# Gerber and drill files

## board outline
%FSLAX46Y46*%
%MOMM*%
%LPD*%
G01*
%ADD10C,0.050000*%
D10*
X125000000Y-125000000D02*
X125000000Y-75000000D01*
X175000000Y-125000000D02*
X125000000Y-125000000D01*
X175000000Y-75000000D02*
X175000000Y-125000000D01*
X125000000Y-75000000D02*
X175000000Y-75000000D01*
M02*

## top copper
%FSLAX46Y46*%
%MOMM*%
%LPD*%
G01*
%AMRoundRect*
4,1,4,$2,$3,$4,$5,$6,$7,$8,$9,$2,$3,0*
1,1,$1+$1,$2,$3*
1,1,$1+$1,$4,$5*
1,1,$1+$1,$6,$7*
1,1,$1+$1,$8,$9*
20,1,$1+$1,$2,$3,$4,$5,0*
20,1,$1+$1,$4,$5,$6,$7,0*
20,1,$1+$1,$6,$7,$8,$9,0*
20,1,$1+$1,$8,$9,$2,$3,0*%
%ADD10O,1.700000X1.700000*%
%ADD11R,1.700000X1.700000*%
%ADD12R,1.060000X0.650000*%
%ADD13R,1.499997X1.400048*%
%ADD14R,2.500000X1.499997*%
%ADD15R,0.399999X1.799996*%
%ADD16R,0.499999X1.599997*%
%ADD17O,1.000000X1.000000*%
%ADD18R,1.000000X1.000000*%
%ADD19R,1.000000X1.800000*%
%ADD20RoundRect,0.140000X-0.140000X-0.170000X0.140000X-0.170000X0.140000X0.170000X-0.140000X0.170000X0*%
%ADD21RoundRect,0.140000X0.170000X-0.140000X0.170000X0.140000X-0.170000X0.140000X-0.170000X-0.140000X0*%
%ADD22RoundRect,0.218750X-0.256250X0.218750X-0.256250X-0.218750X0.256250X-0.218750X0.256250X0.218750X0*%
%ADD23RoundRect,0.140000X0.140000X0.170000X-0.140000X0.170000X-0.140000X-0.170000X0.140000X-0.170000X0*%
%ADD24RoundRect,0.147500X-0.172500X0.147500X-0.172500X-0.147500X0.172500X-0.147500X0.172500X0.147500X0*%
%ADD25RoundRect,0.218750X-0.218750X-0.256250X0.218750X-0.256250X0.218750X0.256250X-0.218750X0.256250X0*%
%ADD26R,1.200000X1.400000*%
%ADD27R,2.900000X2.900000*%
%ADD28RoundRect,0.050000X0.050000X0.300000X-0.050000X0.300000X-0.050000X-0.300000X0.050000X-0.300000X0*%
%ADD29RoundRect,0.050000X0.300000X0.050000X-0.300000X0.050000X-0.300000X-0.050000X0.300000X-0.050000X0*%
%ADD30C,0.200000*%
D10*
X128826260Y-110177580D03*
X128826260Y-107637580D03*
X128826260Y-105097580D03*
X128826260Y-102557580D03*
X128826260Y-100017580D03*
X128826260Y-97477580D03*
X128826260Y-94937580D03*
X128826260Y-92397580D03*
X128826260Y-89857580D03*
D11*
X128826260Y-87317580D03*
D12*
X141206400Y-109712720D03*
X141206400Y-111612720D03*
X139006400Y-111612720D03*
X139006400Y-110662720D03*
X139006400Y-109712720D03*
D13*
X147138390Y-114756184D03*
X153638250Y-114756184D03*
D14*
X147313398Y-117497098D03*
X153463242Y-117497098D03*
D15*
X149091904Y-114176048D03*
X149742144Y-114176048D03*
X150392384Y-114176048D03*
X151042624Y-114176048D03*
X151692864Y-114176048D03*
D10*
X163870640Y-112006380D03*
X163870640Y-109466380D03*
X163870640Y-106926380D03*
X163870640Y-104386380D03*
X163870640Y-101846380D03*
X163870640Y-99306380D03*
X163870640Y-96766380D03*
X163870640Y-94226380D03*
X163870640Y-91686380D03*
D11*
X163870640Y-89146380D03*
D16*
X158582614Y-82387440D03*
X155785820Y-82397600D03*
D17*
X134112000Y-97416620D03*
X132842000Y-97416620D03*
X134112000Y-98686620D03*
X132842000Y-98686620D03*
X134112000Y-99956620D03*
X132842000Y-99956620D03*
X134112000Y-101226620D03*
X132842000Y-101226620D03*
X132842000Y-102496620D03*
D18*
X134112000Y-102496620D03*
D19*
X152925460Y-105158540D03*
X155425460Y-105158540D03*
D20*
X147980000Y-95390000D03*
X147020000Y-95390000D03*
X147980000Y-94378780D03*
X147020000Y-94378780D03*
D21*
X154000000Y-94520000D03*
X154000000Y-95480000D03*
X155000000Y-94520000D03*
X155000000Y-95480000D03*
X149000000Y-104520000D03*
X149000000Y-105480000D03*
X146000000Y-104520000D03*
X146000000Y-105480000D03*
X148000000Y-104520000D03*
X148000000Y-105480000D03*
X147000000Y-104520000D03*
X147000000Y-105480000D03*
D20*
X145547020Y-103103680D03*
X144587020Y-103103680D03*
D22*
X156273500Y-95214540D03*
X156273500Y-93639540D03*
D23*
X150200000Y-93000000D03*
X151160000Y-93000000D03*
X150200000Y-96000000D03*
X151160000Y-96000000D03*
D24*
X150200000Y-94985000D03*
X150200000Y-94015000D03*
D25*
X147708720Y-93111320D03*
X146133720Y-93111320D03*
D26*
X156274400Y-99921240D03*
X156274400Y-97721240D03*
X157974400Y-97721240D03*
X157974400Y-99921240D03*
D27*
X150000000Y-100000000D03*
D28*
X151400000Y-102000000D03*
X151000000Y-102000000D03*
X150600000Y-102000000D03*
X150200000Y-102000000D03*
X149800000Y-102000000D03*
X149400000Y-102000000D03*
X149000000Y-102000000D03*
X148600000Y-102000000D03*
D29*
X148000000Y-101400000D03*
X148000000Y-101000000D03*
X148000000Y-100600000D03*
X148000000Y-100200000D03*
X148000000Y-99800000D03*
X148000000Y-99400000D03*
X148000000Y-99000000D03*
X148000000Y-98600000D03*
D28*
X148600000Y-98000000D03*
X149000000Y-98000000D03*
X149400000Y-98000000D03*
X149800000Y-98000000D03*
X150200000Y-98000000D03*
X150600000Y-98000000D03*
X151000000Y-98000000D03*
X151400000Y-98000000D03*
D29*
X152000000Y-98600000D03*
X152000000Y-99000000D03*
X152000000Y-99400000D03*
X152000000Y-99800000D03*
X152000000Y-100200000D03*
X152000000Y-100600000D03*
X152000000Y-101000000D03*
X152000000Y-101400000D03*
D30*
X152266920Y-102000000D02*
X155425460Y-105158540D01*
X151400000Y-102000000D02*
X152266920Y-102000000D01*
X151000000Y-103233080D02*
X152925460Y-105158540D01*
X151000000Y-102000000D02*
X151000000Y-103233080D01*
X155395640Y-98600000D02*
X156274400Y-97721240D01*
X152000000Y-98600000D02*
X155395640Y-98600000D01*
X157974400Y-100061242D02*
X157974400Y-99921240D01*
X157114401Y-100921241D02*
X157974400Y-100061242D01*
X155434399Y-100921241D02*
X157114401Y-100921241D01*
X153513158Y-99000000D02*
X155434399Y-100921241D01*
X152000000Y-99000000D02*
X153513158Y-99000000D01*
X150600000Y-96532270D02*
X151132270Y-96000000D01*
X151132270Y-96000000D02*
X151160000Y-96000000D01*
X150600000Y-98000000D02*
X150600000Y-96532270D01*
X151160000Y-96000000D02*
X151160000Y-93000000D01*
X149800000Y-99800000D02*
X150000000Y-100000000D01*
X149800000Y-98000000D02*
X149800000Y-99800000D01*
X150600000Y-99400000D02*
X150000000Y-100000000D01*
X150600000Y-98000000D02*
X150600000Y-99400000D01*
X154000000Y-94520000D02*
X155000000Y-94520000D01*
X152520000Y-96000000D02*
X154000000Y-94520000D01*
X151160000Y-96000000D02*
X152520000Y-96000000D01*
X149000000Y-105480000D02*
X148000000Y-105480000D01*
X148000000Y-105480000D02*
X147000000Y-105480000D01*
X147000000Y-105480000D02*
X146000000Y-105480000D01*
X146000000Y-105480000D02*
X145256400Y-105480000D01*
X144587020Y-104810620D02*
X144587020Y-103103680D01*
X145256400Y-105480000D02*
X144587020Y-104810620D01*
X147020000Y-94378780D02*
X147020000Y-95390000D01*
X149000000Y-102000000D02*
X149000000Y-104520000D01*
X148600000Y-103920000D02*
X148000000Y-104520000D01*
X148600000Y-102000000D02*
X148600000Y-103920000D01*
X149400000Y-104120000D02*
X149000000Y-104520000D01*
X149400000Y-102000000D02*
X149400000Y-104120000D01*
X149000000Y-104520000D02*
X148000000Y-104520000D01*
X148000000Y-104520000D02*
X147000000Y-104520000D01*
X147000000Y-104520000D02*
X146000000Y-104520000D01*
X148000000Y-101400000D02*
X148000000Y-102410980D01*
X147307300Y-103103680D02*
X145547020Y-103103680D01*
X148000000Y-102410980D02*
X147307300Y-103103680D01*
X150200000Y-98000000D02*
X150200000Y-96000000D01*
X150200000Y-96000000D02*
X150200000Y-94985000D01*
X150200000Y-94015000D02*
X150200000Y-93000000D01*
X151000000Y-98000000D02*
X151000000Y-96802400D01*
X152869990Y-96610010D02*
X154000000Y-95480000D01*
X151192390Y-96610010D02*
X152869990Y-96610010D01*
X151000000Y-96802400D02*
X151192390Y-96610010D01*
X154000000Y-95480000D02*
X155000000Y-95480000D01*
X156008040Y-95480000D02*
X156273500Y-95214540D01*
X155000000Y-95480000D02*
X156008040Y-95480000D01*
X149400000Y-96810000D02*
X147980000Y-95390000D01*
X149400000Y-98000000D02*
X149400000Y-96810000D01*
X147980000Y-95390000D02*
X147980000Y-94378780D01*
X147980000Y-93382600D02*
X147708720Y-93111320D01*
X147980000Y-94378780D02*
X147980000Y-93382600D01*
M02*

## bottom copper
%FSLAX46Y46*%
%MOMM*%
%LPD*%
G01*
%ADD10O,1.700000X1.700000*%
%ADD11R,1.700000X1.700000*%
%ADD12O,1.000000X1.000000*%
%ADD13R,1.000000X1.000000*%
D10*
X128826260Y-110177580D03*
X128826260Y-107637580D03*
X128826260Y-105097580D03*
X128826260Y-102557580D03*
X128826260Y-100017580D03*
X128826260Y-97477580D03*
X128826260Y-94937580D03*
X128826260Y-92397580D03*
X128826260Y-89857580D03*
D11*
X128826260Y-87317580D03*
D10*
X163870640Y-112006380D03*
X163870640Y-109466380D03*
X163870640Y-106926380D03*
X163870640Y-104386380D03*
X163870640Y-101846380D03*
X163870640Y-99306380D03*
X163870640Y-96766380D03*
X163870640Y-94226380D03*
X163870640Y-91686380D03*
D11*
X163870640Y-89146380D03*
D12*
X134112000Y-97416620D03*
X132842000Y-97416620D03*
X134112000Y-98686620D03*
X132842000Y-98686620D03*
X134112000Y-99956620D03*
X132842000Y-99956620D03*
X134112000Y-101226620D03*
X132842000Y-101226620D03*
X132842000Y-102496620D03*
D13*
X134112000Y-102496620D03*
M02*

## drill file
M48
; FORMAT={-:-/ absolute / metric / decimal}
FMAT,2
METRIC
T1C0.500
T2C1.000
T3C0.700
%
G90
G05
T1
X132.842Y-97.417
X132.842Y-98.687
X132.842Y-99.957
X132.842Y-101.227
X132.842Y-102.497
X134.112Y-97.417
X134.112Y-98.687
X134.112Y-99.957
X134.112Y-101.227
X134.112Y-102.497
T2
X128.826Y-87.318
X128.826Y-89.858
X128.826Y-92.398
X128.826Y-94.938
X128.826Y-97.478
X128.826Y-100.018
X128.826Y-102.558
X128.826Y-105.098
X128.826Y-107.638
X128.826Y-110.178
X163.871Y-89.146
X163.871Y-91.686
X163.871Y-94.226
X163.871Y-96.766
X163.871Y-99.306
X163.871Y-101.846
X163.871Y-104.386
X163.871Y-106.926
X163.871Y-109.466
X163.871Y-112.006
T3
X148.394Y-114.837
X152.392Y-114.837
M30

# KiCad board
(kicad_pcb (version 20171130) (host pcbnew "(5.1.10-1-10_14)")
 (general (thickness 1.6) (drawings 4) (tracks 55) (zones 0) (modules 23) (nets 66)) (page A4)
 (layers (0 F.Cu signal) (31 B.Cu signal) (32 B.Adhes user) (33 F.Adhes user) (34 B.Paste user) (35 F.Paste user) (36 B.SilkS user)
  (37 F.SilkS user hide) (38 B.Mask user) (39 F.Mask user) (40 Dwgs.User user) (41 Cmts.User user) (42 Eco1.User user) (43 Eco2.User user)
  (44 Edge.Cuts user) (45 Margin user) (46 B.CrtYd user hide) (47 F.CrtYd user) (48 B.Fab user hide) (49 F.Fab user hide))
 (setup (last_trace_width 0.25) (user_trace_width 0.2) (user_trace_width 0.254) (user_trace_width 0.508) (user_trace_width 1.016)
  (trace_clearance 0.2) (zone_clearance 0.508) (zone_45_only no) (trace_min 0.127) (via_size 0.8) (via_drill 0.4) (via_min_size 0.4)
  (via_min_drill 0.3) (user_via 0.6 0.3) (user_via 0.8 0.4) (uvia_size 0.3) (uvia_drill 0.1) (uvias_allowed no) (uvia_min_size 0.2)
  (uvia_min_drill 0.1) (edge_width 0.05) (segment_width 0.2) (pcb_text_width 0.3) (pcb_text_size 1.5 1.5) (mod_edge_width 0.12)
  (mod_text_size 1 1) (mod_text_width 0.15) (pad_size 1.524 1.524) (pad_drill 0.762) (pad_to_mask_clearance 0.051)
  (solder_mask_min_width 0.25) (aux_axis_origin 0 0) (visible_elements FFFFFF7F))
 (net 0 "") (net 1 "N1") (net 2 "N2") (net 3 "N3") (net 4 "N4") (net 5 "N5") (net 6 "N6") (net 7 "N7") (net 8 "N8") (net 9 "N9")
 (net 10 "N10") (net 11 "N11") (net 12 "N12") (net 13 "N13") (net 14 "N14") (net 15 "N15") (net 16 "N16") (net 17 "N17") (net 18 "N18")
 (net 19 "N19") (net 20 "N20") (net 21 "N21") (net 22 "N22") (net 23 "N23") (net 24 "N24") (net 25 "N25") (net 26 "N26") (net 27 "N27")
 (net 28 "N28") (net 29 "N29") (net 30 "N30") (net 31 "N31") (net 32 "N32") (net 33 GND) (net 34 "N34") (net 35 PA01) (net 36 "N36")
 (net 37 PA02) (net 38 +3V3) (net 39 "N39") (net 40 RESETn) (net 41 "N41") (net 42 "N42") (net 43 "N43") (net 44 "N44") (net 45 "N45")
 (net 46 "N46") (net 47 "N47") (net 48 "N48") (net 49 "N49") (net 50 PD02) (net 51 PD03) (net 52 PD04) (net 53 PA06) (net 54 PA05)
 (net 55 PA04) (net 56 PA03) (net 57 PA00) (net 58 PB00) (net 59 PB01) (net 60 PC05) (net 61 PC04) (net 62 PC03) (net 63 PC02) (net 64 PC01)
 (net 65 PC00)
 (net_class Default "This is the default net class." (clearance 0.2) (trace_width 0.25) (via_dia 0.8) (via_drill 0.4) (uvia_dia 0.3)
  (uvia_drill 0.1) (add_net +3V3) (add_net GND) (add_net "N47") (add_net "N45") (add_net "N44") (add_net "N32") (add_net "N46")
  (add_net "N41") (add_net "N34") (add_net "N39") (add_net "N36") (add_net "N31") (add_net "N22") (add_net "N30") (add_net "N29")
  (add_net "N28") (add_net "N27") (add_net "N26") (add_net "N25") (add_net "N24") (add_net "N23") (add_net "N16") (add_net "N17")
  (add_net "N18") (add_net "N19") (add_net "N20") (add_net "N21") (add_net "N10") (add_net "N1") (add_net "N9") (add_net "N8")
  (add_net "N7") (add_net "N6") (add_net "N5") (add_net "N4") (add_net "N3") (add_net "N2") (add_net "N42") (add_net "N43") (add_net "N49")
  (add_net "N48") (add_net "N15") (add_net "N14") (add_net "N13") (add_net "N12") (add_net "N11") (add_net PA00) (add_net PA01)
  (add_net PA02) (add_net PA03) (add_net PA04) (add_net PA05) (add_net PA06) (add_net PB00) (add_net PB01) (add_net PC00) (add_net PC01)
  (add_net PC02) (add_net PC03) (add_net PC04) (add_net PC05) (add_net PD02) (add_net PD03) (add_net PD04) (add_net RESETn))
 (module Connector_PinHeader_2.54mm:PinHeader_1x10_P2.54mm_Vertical (layer F.Cu) (at 128.82626 87.31758)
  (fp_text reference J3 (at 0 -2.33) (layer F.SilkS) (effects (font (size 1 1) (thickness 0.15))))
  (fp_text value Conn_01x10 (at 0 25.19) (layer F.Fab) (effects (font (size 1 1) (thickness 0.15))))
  (pad 10 thru_hole oval (at 0 22.86) (size 1.7 1.7) (drill 1) (layers *.Cu *.Mask) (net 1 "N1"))
  (pad 9 thru_hole oval (at 0 20.32) (size 1.7 1.7) (drill 1) (layers *.Cu *.Mask) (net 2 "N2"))
  (pad 8 thru_hole oval (at 0 17.78) (size 1.7 1.7) (drill 1) (layers *.Cu *.Mask) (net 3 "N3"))
  (pad 7 thru_hole oval (at 0 15.24) (size 1.7 1.7) (drill 1) (layers *.Cu *.Mask) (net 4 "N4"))
  (pad 6 thru_hole oval (at 0 12.7) (size 1.7 1.7) (drill 1) (layers *.Cu *.Mask) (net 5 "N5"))
  (pad 5 thru_hole oval (at 0 10.16) (size 1.7 1.7) (drill 1) (layers *.Cu *.Mask) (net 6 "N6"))
  (pad 4 thru_hole oval (at 0 7.62) (size 1.7 1.7) (drill 1) (layers *.Cu *.Mask) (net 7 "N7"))
  (pad 3 thru_hole oval (at 0 5.08) (size 1.7 1.7) (drill 1) (layers *.Cu *.Mask) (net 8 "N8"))
  (pad 2 thru_hole oval (at 0 2.54) (size 1.7 1.7) (drill 1) (layers *.Cu *.Mask) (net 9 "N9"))
  (pad 1 thru_hole rect (at 0 0) (size 1.7 1.7) (drill 1) (layers *.Cu *.Mask) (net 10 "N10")))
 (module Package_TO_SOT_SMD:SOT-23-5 (layer F.Cu) (at 140.1064 110.66272)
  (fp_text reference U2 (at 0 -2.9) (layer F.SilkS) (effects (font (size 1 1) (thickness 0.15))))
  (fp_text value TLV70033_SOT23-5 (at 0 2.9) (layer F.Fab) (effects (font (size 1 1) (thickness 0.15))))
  (pad 5 smd rect (at 1.1 -0.95) (size 1.06 0.65) (layers F.Cu F.Paste F.Mask) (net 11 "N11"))
  (pad 4 smd rect (at 1.1 0.95) (size 1.06 0.65) (layers F.Cu F.Paste F.Mask) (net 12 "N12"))
  (pad 3 smd rect (at -1.1 0.95) (size 1.06 0.65) (layers F.Cu F.Paste F.Mask) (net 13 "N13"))
  (pad 2 smd rect (at -1.1 0) (size 1.06 0.65) (layers F.Cu F.Paste F.Mask) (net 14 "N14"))
  (pad 1 smd rect (at -1.1 -0.95) (size 1.06 0.65) (layers F.Cu F.Paste F.Mask) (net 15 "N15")))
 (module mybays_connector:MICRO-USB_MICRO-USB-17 (layer F.Cu) (at 150.38832 115.8367 180)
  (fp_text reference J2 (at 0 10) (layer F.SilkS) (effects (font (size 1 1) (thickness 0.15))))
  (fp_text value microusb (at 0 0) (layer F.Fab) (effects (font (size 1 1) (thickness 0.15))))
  (pad 0 smd rect (at 3.24993 1.080516 180) (size 1.499997 1.400048) (layers F.Cu F.Paste F.Mask) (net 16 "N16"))
  (pad 0 smd rect (at -3.24993 1.080516 180) (size 1.499997 1.400048) (layers F.Cu F.Paste F.Mask) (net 16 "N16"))
  (pad 0 smd rect (at 3.074922 -1.660398) (size 2.5 1.499997) (layers F.Cu F.Paste F.Mask) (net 16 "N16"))
  (pad 0 smd rect (at -3.074922 -1.660398 90) (size 1.499997 2.5) (layers F.Cu F.Paste F.Mask) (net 16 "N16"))
  (pad 1 smd rect (at 1.296416 1.660652 270) (size 1.799996 0.399999) (layers F.Cu F.Paste F.Mask) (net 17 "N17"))
  (pad 2 smd rect (at 0.646176 1.660652 270) (size 1.799996 0.399999) (layers F.Cu F.Paste F.Mask) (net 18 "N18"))
  (pad 3 smd rect (at -0.004064 1.660652 270) (size 1.799996 0.399999) (layers F.Cu F.Paste F.Mask) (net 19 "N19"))
  (pad 4 smd rect (at -0.654304 1.660652 270) (size 1.799996 0.399999) (layers F.Cu F.Paste F.Mask) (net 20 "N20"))
  (pad 5 smd rect (at -1.304544 1.660652 270) (size 1.799996 0.399999) (layers F.Cu F.Paste F.Mask) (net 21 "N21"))
  (pad "" np_thru_hole circle (at 1.9939 0.999236 180) (size 0.700024 0.700024) (drill 0.700024) (layers *.Cu *.Mask))
  (pad "" np_thru_hole circle (at -2.00406 0.999236 180) (size 0.700024 0.700024) (drill 0.700024) (layers *.Cu *.Mask)))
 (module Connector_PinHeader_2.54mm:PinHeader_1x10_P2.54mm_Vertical (layer F.Cu) (at 163.87064 89.14638)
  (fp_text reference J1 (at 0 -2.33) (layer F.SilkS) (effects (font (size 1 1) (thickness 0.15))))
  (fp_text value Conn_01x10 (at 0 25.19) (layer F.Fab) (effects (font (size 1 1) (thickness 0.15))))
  (pad 10 thru_hole oval (at 0 22.86) (size 1.7 1.7) (drill 1) (layers *.Cu *.Mask) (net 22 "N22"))
  (pad 9 thru_hole oval (at 0 20.32) (size 1.7 1.7) (drill 1) (layers *.Cu *.Mask) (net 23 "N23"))
  (pad 8 thru_hole oval (at 0 17.78) (size 1.7 1.7) (drill 1) (layers *.Cu *.Mask) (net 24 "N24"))
  (pad 7 thru_hole oval (at 0 15.24) (size 1.7 1.7) (drill 1) (layers *.Cu *.Mask) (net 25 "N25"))
  (pad 6 thru_hole oval (at 0 12.7) (size 1.7 1.7) (drill 1) (layers *.Cu *.Mask) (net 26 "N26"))
  (pad 5 thru_hole oval (at 0 10.16) (size 1.7 1.7) (drill 1) (layers *.Cu *.Mask) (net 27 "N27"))
  (pad 4 thru_hole oval (at 0 7.62) (size 1.7 1.7) (drill 1) (layers *.Cu *.Mask) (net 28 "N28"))
  (pad 3 thru_hole oval (at 0 5.08) (size 1.7 1.7) (drill 1) (layers *.Cu *.Mask) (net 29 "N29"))
  (pad 2 thru_hole oval (at 0 2.54) (size 1.7 1.7) (drill 1) (layers *.Cu *.Mask) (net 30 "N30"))
  (pad 1 thru_hole rect (at 0 0) (size 1.7 1.7) (drill 1) (layers *.Cu *.Mask) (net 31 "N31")))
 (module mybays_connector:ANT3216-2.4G (layer F.Cu) (at 155.58516 83.19008)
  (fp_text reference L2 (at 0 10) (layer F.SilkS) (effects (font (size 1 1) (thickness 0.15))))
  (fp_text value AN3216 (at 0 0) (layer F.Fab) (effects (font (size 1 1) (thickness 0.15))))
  (pad "" smd rect (at 2.997454 -0.80264) (size 0.499999 1.599997) (layers F.Cu F.Paste F.Mask))
  (pad 1 smd rect (at 0.20066 -0.79248) (size 0.499999 1.599997) (layers F.Cu F.Paste F.Mask) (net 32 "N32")))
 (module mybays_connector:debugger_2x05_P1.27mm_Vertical (layer F.Cu) (at 133.477 99.95662 180)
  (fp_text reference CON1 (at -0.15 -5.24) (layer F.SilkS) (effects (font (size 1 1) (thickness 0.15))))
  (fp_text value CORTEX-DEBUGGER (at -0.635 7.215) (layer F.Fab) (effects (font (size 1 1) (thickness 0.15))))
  (pad 9 thru_hole oval (at -0.635 2.54 180) (size 1 1) (drill 0.5) (layers *.Cu *.Mask) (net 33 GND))
  (pad 10 thru_hole oval (at 0.635 2.54 180) (size 1 1) (drill 0.5) (layers *.Cu *.Mask) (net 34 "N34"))
  (pad 7 thru_hole oval (at -0.635 1.27 180) (size 1 1) (drill 0.5) (layers *.Cu *.Mask) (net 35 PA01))
  (pad 8 thru_hole oval (at 0.635 1.27 180) (size 1 1) (drill 0.5) (layers *.Cu *.Mask) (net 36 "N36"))
  (pad 5 thru_hole oval (at -0.635 0 180) (size 1 1) (drill 0.5) (layers *.Cu *.Mask) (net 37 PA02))
  (pad 6 thru_hole oval (at 0.635 0 180) (size 1 1) (drill 0.5) (layers *.Cu *.Mask) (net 33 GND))
  (pad 3 thru_hole oval (at -0.635 -1.27 180) (size 1 1) (drill 0.5) (layers *.Cu *.Mask) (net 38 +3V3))
  (pad 4 thru_hole oval (at 0.635 -1.27 180) (size 1 1) (drill 0.5) (layers *.Cu *.Mask) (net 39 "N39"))
  (pad 2 thru_hole oval (at 0.635 -2.54 180) (size 1 1) (drill 0.5) (layers *.Cu *.Mask) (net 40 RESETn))
  (pad 1 thru_hole rect (at -0.635 -2.54 180) (size 1 1) (drill 0.5) (layers *.Cu *.Mask) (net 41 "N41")))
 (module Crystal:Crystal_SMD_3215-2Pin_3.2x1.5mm (layer F.Cu) (at 154.17546 105.15854)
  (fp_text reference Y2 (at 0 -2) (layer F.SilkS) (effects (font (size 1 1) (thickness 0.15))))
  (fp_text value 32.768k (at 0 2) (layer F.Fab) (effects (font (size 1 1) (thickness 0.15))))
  (pad 2 smd rect (at -1.25 0) (size 1 1.8) (layers F.Cu F.Paste F.Mask) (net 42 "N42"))
  (pad 1 smd rect (at 1.25 0) (size 1 1.8) (layers F.Cu F.Paste F.Mask) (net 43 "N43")))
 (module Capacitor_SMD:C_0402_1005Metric (layer F.Cu) (at 147.5 95.39)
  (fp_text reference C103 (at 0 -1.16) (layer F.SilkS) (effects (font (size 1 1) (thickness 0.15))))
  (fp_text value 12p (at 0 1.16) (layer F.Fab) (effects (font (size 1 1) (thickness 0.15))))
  (pad 2 smd roundrect (at 0.48 0) (size 0.56 0.62) (layers F.Cu F.Paste F.Mask) (roundrect_rratio 0.25) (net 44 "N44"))
  (pad 1 smd roundrect (at -0.48 0) (size 0.56 0.62) (layers F.Cu F.Paste F.Mask) (roundrect_rratio 0.25) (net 33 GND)))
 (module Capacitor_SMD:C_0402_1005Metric (layer F.Cu) (at 147.5 94.37878)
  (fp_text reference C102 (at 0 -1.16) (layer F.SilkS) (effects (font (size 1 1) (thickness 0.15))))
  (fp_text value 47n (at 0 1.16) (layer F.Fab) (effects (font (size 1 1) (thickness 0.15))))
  (pad 2 smd roundrect (at 0.48 0) (size 0.56 0.62) (layers F.Cu F.Paste F.Mask) (roundrect_rratio 0.25) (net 44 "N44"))
  (pad 1 smd roundrect (at -0.48 0) (size 0.56 0.62) (layers F.Cu F.Paste F.Mask) (roundrect_rratio 0.25) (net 33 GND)))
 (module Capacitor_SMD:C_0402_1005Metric (layer F.Cu) (at 154 95 90)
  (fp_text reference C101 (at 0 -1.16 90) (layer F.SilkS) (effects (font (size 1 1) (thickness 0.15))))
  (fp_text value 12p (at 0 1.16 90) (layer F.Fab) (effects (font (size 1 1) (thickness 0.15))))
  (pad 2 smd roundrect (at 0.48 0 90) (size 0.56 0.62) (layers F.Cu F.Paste F.Mask) (roundrect_rratio 0.25) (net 33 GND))
  (pad 1 smd roundrect (at -0.48 0 90) (size 0.56 0.62) (layers F.Cu F.Paste F.Mask) (roundrect_rratio 0.25) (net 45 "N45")))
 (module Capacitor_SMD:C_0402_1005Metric (layer F.Cu) (at 155 95 90)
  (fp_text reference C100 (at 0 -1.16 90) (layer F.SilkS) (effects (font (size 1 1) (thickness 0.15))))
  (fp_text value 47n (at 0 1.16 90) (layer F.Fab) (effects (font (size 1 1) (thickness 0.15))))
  (pad 2 smd roundrect (at 0.48 0 90) (size 0.56 0.62) (layers F.Cu F.Paste F.Mask) (roundrect_rratio 0.25) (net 33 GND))
  (pad 1 smd roundrect (at -0.48 0 90) (size 0.56 0.62) (layers F.Cu F.Paste F.Mask) (roundrect_rratio 0.25) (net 45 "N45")))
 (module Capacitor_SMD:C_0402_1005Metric (layer F.Cu) (at 149 105 90)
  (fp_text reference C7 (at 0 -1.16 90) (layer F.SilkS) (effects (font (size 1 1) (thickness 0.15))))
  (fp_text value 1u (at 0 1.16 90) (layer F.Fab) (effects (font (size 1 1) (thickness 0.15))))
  (pad 2 smd roundrect (at 0.48 0 90) (size 0.56 0.62) (layers F.Cu F.Paste F.Mask) (roundrect_rratio 0.25) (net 38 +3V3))
  (pad 1 smd roundrect (at -0.48 0 90) (size 0.56 0.62) (layers F.Cu F.Paste F.Mask) (roundrect_rratio 0.25) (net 33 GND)))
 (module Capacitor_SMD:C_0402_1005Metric (layer F.Cu) (at 146 105 90)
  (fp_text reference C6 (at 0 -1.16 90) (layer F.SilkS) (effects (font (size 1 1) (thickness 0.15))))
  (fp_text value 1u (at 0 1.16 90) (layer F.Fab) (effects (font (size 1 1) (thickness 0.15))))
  (pad 2 smd roundrect (at 0.48 0 90) (size 0.56 0.62) (layers F.Cu F.Paste F.Mask) (roundrect_rratio 0.25) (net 38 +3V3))
  (pad 1 smd roundrect (at -0.48 0 90) (size 0.56 0.62) (layers F.Cu F.Paste F.Mask) (roundrect_rratio 0.25) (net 33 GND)))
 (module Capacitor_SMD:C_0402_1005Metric (layer F.Cu) (at 148 105 90)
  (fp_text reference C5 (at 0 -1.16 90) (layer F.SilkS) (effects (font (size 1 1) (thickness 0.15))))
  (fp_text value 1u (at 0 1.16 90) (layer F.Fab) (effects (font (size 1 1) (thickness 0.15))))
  (pad 2 smd roundrect (at 0.48 0 90) (size 0.56 0.62) (layers F.Cu F.Paste F.Mask) (roundrect_rratio 0.25) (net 38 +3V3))
  (pad 1 smd roundrect (at -0.48 0 90) (size 0.56 0.62) (layers F.Cu F.Paste F.Mask) (roundrect_rratio 0.25) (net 33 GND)))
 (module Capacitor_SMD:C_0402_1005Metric (layer F.Cu) (at 147 105 90)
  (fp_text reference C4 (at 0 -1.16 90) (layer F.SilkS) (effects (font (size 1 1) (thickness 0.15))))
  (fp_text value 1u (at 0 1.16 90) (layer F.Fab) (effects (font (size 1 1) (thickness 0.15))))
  (pad 2 smd roundrect (at 0.48 0 90) (size 0.56 0.62) (layers F.Cu F.Paste F.Mask) (roundrect_rratio 0.25) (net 38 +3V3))
  (pad 1 smd roundrect (at -0.48 0 90) (size 0.56 0.62) (layers F.Cu F.Paste F.Mask) (roundrect_rratio 0.25) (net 33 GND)))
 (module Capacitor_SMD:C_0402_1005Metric (layer F.Cu) (at 145.06702 103.10368)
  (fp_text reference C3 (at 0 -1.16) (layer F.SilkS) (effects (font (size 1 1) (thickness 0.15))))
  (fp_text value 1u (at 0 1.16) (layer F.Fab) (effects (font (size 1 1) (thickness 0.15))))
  (pad 2 smd roundrect (at 0.48 0) (size 0.56 0.62) (layers F.Cu F.Paste F.Mask) (roundrect_rratio 0.25) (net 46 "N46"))
  (pad 1 smd roundrect (at -0.48 0) (size 0.56 0.62) (layers F.Cu F.Paste F.Mask) (roundrect_rratio 0.25) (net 33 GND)))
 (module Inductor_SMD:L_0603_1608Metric (layer F.Cu) (at 156.2735 94.42704 270)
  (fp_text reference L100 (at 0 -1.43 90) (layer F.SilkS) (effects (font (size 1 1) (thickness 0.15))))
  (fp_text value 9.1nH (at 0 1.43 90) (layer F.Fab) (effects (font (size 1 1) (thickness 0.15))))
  (pad 2 smd roundrect (at 0.7875 0 270) (size 0.875 0.95) (layers F.Cu F.Paste F.Mask) (roundrect_rratio 0.25) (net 45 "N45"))
  (pad 1 smd roundrect (at -0.7875 0 270) (size 0.875 0.95) (layers F.Cu F.Paste F.Mask) (roundrect_rratio 0.25) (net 38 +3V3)))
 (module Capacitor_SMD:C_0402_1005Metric (layer F.Cu) (at 150.68 93 180)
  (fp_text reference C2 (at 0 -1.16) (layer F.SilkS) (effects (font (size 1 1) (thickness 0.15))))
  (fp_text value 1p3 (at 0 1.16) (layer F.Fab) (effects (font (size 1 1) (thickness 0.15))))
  (pad 2 smd roundrect (at 0.48 0 180) (size 0.56 0.62) (layers F.Cu F.Paste F.Mask) (roundrect_rratio 0.25) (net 32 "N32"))
  (pad 1 smd roundrect (at -0.48 0 180) (size 0.56 0.62) (layers F.Cu F.Paste F.Mask) (roundrect_rratio 0.25) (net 33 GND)))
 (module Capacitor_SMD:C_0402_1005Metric (layer F.Cu) (at 150.68 96 180)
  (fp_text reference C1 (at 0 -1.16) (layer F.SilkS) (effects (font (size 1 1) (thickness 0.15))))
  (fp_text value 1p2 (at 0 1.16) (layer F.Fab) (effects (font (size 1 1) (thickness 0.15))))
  (pad 2 smd roundrect (at 0.48 0 180) (size 0.56 0.62) (layers F.Cu F.Paste F.Mask) (roundrect_rratio 0.25) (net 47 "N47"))
  (pad 1 smd roundrect (at -0.48 0 180) (size 0.56 0.62) (layers F.Cu F.Paste F.Mask) (roundrect_rratio 0.25) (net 33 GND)))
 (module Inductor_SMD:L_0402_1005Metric (layer F.Cu) (at 150.2 94.5 270)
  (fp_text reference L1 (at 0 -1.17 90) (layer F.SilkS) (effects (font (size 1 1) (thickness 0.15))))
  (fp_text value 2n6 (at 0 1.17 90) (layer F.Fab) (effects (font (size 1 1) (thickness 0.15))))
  (pad 2 smd roundrect (at 0.485 0 270) (size 0.59 0.64) (layers F.Cu F.Paste F.Mask) (roundrect_rratio 0.25) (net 47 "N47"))
  (pad 1 smd roundrect (at -0.485 0 270) (size 0.59 0.64) (layers F.Cu F.Paste F.Mask) (roundrect_rratio 0.25) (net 32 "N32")))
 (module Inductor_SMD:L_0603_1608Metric (layer F.Cu) (at 146.92122 93.11132)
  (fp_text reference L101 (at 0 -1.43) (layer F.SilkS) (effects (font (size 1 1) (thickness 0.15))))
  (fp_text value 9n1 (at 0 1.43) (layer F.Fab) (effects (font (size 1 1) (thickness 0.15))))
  (pad 2 smd roundrect (at 0.7875 0) (size 0.875 0.95) (layers F.Cu F.Paste F.Mask) (roundrect_rratio 0.25) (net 44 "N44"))
  (pad 1 smd roundrect (at -0.7875 0) (size 0.875 0.95) (layers F.Cu F.Paste F.Mask) (roundrect_rratio 0.25) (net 38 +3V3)))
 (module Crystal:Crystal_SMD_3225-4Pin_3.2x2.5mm (layer F.Cu) (at 157.1244 98.82124 90)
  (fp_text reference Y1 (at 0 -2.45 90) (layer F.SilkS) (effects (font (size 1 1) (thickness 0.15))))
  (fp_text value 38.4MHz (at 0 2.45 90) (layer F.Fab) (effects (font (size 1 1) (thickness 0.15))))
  (pad 4 smd rect (at -1.1 -0.85 90) (size 1.4 1.2) (layers F.Cu F.Paste F.Mask) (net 33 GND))
  (pad 3 smd rect (at 1.1 -0.85 90) (size 1.4 1.2) (layers F.Cu F.Paste F.Mask) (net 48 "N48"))
  (pad 2 smd rect (at 1.1 0.85 90) (size 1.4 1.2) (layers F.Cu F.Paste F.Mask) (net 33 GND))
  (pad 1 smd rect (at -1.1 0.85 90) (size 1.4 1.2) (layers F.Cu F.Paste F.Mask) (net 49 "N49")))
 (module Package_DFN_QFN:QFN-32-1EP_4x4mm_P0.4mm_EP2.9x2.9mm (layer F.Cu) (at 150 100 180)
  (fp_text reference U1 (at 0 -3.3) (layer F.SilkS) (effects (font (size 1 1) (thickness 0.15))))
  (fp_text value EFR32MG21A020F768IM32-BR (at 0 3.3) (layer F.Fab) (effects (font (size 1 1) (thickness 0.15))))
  (pad "" smd roundrect (at 0.725 0.725 180) (size 1.17 1.17) (layers F.Paste) (roundrect_rratio 0.213675))
  (pad "" smd roundrect (at 0.725 -0.725 180) (size 1.17 1.17) (layers F.Paste) (roundrect_rratio 0.213675))
  (pad "" smd roundrect (at -0.725 0.725 180) (size 1.17 1.17) (layers F.Paste) (roundrect_rratio 0.213675))
  (pad "" smd roundrect (at -0.725 -0.725 180) (size 1.17 1.17) (layers F.Paste) (roundrect_rratio 0.213675))
  (pad 33 smd rect (at 0 0 180) (size 2.9 2.9) (layers F.Cu F.Mask) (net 33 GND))
  (pad 32 smd roundrect (at -1.4 -2 180) (size 0.2 0.7) (layers F.Cu F.Paste F.Mask) (roundrect_rratio 0.25) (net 43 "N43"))
  (pad 31 smd roundrect (at -1 -2 180) (size 0.2 0.7) (layers F.Cu F.Paste F.Mask) (roundrect_rratio 0.25) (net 42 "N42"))
  (pad 30 smd roundrect (at -0.6 -2 180) (size 0.2 0.7) (layers F.Cu F.Paste F.Mask) (roundrect_rratio 0.25) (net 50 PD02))
  (pad 29 smd roundrect (at -0.2 -2 180) (size 0.2 0.7) (layers F.Cu F.Paste F.Mask) (roundrect_rratio 0.25) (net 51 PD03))
  (pad 28 smd roundrect (at 0.2 -2 180) (size 0.2 0.7) (layers F.Cu F.Paste F.Mask) (roundrect_rratio 0.25) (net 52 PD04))
  (pad 27 smd roundrect (at 0.6 -2 180) (size 0.2 0.7) (layers F.Cu F.Paste F.Mask) (roundrect_rratio 0.25) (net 38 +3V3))
  (pad 26 smd roundrect (at 1 -2 180) (size 0.2 0.7) (layers F.Cu F.Paste F.Mask) (roundrect_rratio 0.25) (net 38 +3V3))
  (pad 25 smd roundrect (at 1.4 -2 180) (size 0.2 0.7) (layers F.Cu F.Paste F.Mask) (roundrect_rratio 0.25) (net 38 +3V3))
  (pad 24 smd roundrect (at 2 -1.4 180) (size 0.7 0.2) (layers F.Cu F.Paste F.Mask) (roundrect_rratio 0.25) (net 46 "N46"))
  (pad 23 smd roundrect (at 2 -1 180) (size 0.7 0.2) (layers F.Cu F.Paste F.Mask) (roundrect_rratio 0.25) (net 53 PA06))
  (pad 22 smd roundrect (at 2 -0.6 180) (size 0.7 0.2) (layers F.Cu F.Paste F.Mask) (roundrect_rratio 0.25) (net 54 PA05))
  (pad 21 smd roundrect (at 2 -0.2 180) (size 0.7 0.2) (layers F.Cu F.Paste F.Mask) (roundrect_rratio 0.25) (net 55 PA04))
  (pad 20 smd roundrect (at 2 0.2 180) (size 0.7 0.2) (layers F.Cu F.Paste F.Mask) (roundrect_rratio 0.25) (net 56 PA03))
  (pad 19 smd roundrect (at 2 0.6 180) (size 0.7 0.2) (layers F.Cu F.Paste F.Mask) (roundrect_rratio 0.25) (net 37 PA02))
  (pad 18 smd roundrect (at 2 1 180) (size 0.7 0.2) (layers F.Cu F.Paste F.Mask) (roundrect_rratio 0.25) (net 35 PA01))
  (pad 17 smd roundrect (at 2 1.4 180) (size 0.7 0.2) (layers F.Cu F.Paste F.Mask) (roundrect_rratio 0.25) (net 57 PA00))
  (pad 16 smd roundrect (at 1.4 2 180) (size 0.2 0.7) (layers F.Cu F.Paste F.Mask) (roundrect_rratio 0.25) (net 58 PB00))
  (pad 15 smd roundrect (at 1 2 180) (size 0.2 0.7) (layers F.Cu F.Paste F.Mask) (roundrect_rratio 0.25) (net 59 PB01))
  (pad 14 smd roundrect (at 0.6 2 180) (size 0.2 0.7) (layers F.Cu F.Paste F.Mask) (roundrect_rratio 0.25) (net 44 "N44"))
  (pad 13 smd roundrect (at 0.2 2 180) (size 0.2 0.7) (layers F.Cu F.Paste F.Mask) (roundrect_rratio 0.25) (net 33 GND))
  (pad 12 smd roundrect (at -0.2 2 180) (size 0.2 0.7) (layers F.Cu F.Paste F.Mask) (roundrect_rratio 0.25) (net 47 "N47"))
  (pad 11 smd roundrect (at -0.6 2 180) (size 0.2 0.7) (layers F.Cu F.Paste F.Mask) (roundrect_rratio 0.25) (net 33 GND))
  (pad 10 smd roundrect (at -1 2 180) (size 0.2 0.7) (layers F.Cu F.Paste F.Mask) (roundrect_rratio 0.25) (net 45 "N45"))
  (pad 9 smd roundrect (at -1.4 2 180) (size 0.2 0.7) (layers F.Cu F.Paste F.Mask) (roundrect_rratio 0.25) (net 40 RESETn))
  (pad 8 smd roundrect (at -2 1.4 180) (size 0.7 0.2) (layers F.Cu F.Paste F.Mask) (roundrect_rratio 0.25) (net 48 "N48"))
  (pad 7 smd roundrect (at -2 1 180) (size 0.7 0.2) (layers F.Cu F.Paste F.Mask) (roundrect_rratio 0.25) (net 49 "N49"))
  (pad 6 smd roundrect (at -2 0.6 180) (size 0.7 0.2) (layers F.Cu F.Paste F.Mask) (roundrect_rratio 0.25) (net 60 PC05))
  (pad 5 smd roundrect (at -2 0.2 180) (size 0.7 0.2) (layers F.Cu F.Paste F.Mask) (roundrect_rratio 0.25) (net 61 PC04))
  (pad 4 smd roundrect (at -2 -0.2 180) (size 0.7 0.2) (layers F.Cu F.Paste F.Mask) (roundrect_rratio 0.25) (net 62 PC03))
  (pad 3 smd roundrect (at -2 -0.6 180) (size 0.7 0.2) (layers F.Cu F.Paste F.Mask) (roundrect_rratio 0.25) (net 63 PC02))
  (pad 2 smd roundrect (at -2 -1 180) (size 0.7 0.2) (layers F.Cu F.Paste F.Mask) (roundrect_rratio 0.25) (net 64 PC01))
  (pad 1 smd roundrect (at -2 -1.4 180) (size 0.7 0.2) (layers F.Cu F.Paste F.Mask) (roundrect_rratio 0.25) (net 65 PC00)))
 (gr_line (start 125 125) (end 125 75) (layer Edge.Cuts) (width 0.05))
 (gr_line (start 175 125) (end 125 125) (layer Edge.Cuts) (width 0.05))
 (gr_line (start 175 75) (end 175 125) (layer Edge.Cuts) (width 0.05))
 (gr_line (start 125 75) (end 175 75) (layer Edge.Cuts) (width 0.05))
 (segment (start 152.26692 102) (end 155.42546 105.15854) (width 0.2) (layer F.Cu) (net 43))
 (segment (start 151.4 102) (end 152.26692 102) (width 0.2) (layer F.Cu) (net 43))
 (segment (start 151 103.23308) (end 152.92546 105.15854) (width 0.2) (layer F.Cu) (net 42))
 (segment (start 151 102) (end 151 103.23308) (width 0.2) (layer F.Cu) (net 42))
 (segment (start 155.39564 98.6) (end 156.2744 97.72124) (width 0.2) (layer F.Cu) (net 48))
 (segment (start 152 98.6) (end 155.39564 98.6) (width 0.2) (layer F.Cu) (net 48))
 (segment (start 157.9744 100.061242) (end 157.9744 99.92124) (width 0.2) (layer F.Cu) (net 49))
 (segment (start 157.114401 100.921241) (end 157.9744 100.061242) (width 0.2) (layer F.Cu) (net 49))
 (segment (start 155.434399 100.921241) (end 157.114401 100.921241) (width 0.2) (layer F.Cu) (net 49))
 (segment (start 153.513158 99) (end 155.434399 100.921241) (width 0.2) (layer F.Cu) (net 49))
 (segment (start 152 99) (end 153.513158 99) (width 0.2) (layer F.Cu) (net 49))
 (segment (start 150.6 96.53227) (end 151.13227 96) (width 0.2) (layer F.Cu) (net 33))
 (segment (start 151.13227 96) (end 151.16 96) (width 0.2) (layer F.Cu) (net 33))
 (segment (start 150.6 98) (end 150.6 96.53227) (width 0.2) (layer F.Cu) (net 33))
 (segment (start 151.16 96) (end 151.16 93) (width 0.2) (layer F.Cu) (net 33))
 (segment (start 149.8 99.8) (end 150 100) (width 0.2) (layer F.Cu) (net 33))
 (segment (start 149.8 98) (end 149.8 99.8) (width 0.2) (layer F.Cu) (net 33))
 (segment (start 150.6 99.4) (end 150 100) (width 0.2) (layer F.Cu) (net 33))
 (segment (start 150.6 98) (end 150.6 99.4) (width 0.2) (layer F.Cu) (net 33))
 (segment (start 154 94.52) (end 155 94.52) (width 0.2) (layer F.Cu) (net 33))
 (segment (start 152.52 96) (end 154 94.52) (width 0.2) (layer F.Cu) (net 33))
 (segment (start 151.16 96) (end 152.52 96) (width 0.2) (layer F.Cu) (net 33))
 (segment (start 149 105.48) (end 148 105.48) (width 0.2) (layer F.Cu) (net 33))
 (segment (start 148 105.48) (end 147 105.48) (width 0.2) (layer F.Cu) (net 33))
 (segment (start 147 105.48) (end 146 105.48) (width 0.2) (layer F.Cu) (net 33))
 (segment (start 146 105.48) (end 145.2564 105.48) (width 0.2) (layer F.Cu) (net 33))
 (segment (start 144.58702 104.81062) (end 144.58702 103.10368) (width 0.2) (layer F.Cu) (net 33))
 (segment (start 145.2564 105.48) (end 144.58702 104.81062) (width 0.2) (layer F.Cu) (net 33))
 (segment (start 147.02 94.37878) (end 147.02 95.39) (width 0.2) (layer F.Cu) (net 33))
 (segment (start 149 102) (end 149 104.52) (width 0.2) (layer F.Cu) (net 38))
 (segment (start 148.6 103.92) (end 148 104.52) (width 0.2) (layer F.Cu) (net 38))
 (segment (start 148.6 102) (end 148.6 103.92) (width 0.2) (layer F.Cu) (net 38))
 (segment (start 149.4 104.12) (end 149 104.52) (width 0.2) (layer F.Cu) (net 38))
 (segment (start 149.4 102) (end 149.4 104.12) (width 0.2) (layer F.Cu) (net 38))
 (segment (start 149 104.52) (end 148 104.52) (width 0.2) (layer F.Cu) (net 38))
 (segment (start 148 104.52) (end 147 104.52) (width 0.2) (layer F.Cu) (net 38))
 (segment (start 147 104.52) (end 146 104.52) (width 0.2) (layer F.Cu) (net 38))
 (segment (start 148 101.4) (end 148 102.41098) (width 0.2) (layer F.Cu) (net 46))
 (segment (start 147.3073 103.10368) (end 145.54702 103.10368) (width 0.2) (layer F.Cu) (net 46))
 (segment (start 148 102.41098) (end 147.3073 103.10368) (width 0.2) (layer F.Cu) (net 46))
 (segment (start 150.2 98) (end 150.2 96) (width 0.2) (layer F.Cu) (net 47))
 (segment (start 150.2 96) (end 150.2 94.985) (width 0.2) (layer F.Cu) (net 47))
 (segment (start 150.2 94.015) (end 150.2 93) (width 0.2) (layer F.Cu) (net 32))
 (segment (start 151 98) (end 151 96.8024) (width 0.2) (layer F.Cu) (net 45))
 (segment (start 152.86999 96.61001) (end 154 95.48) (width 0.2) (layer F.Cu) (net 45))
 (segment (start 151.19239 96.61001) (end 152.86999 96.61001) (width 0.2) (layer F.Cu) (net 45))
 (segment (start 151 96.8024) (end 151.19239 96.61001) (width 0.2) (layer F.Cu) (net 45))
 (segment (start 154 95.48) (end 155 95.48) (width 0.2) (layer F.Cu) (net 45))
 (segment (start 156.00804 95.48) (end 156.2735 95.21454) (width 0.2) (layer F.Cu) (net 45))
 (segment (start 155 95.48) (end 156.00804 95.48) (width 0.2) (layer F.Cu) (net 45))
 (segment (start 149.4 96.81) (end 147.98 95.39) (width 0.2) (layer F.Cu) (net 44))
 (segment (start 149.4 98) (end 149.4 96.81) (width 0.2) (layer F.Cu) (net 44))
 (segment (start 147.98 95.39) (end 147.98 94.37878) (width 0.2) (layer F.Cu) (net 44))
 (segment (start 147.98 93.3826) (end 147.70872 93.11132) (width 0.2) (layer F.Cu) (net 44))
 (segment (start 147.98 94.37878) (end 147.98 93.3826) (width 0.2) (layer F.Cu) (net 44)))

